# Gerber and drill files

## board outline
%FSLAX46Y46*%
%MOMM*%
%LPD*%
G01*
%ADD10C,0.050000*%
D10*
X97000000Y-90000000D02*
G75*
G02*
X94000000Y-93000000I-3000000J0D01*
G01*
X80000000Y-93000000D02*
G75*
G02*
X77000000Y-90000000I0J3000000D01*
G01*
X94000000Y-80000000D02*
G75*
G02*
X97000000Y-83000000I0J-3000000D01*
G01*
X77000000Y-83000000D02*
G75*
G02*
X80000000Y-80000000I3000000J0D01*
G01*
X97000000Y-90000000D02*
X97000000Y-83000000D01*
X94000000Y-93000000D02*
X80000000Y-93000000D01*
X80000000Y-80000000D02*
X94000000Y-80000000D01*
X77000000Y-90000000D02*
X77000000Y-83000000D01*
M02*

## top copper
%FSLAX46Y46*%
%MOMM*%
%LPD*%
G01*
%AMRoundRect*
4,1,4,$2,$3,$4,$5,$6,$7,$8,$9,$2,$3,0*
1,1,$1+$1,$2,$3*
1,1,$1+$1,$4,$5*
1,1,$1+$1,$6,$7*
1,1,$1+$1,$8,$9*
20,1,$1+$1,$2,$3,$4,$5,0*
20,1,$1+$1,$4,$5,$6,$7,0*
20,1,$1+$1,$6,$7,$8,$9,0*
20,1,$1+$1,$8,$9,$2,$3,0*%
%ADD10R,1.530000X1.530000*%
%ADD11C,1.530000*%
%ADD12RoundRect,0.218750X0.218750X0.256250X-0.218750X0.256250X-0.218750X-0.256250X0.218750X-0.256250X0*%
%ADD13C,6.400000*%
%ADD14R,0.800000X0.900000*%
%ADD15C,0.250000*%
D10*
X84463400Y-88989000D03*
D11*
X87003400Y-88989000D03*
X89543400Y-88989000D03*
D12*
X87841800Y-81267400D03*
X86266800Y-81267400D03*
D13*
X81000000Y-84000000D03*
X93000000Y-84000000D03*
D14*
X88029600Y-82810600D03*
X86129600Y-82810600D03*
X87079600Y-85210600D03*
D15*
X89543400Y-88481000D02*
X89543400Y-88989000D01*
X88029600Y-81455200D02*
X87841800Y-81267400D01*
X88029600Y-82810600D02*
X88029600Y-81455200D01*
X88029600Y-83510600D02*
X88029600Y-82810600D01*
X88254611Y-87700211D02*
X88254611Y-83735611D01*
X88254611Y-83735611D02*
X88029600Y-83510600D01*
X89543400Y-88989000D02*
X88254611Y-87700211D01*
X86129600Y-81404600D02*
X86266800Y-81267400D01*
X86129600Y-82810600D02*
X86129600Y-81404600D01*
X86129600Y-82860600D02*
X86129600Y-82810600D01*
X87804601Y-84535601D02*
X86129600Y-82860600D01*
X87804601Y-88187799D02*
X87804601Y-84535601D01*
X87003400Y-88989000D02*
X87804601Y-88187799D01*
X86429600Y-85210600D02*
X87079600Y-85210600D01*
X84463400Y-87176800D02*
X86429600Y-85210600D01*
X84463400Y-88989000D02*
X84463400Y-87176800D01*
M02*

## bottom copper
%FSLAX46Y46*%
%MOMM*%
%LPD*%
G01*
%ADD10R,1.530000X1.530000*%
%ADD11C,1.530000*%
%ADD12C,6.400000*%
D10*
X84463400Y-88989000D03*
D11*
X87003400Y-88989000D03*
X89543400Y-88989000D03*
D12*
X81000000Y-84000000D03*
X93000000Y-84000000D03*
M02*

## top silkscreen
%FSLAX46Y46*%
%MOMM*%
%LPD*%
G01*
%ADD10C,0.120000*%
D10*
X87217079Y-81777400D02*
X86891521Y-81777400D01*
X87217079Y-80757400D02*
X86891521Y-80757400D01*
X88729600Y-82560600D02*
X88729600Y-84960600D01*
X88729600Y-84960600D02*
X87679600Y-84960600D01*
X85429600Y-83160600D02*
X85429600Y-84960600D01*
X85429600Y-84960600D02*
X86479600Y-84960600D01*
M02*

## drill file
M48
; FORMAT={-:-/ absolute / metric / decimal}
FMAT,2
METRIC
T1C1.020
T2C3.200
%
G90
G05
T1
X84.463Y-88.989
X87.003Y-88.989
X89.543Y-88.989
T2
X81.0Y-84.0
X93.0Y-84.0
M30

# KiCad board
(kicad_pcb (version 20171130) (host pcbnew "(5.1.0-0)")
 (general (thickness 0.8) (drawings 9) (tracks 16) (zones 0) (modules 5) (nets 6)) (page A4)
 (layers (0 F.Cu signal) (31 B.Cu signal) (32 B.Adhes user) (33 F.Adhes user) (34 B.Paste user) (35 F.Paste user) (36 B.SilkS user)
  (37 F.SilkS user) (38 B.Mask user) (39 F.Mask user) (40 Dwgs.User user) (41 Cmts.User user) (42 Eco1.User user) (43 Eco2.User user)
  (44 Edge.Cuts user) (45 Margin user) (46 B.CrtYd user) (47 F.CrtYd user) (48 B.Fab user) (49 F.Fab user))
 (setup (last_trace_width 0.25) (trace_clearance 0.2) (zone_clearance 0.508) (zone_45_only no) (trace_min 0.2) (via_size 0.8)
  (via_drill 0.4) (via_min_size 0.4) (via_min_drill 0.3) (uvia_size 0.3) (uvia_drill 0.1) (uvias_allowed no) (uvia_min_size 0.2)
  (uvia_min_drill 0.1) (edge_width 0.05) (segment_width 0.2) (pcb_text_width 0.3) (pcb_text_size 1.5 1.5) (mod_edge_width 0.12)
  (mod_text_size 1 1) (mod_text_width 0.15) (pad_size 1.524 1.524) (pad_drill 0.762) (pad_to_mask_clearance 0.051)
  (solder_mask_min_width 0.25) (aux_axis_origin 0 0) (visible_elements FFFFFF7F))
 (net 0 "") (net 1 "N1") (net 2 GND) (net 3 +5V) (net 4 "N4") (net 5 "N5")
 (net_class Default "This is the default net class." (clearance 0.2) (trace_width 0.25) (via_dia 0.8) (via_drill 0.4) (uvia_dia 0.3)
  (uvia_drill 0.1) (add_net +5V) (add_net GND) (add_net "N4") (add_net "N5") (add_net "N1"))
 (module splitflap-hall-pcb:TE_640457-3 (layer B.Cu) (at 84.4634 88.989 180)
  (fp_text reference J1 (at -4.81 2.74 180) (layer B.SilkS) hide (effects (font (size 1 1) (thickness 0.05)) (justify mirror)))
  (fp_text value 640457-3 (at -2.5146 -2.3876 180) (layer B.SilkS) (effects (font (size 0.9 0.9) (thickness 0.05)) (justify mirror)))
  (pad 1 thru_hole rect (at 0 0 180) (size 1.53 1.53) (drill 1.02) (layers *.Cu *.Mask) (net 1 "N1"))
  (pad 2 thru_hole circle (at -2.54 0 180) (size 1.53 1.53) (drill 1.02) (layers *.Cu *.Mask) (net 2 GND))
  (pad 3 thru_hole circle (at -5.08 0 180) (size 1.53 1.53) (drill 1.02) (layers *.Cu *.Mask) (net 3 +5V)))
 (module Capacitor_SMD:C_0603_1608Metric (layer F.Cu) (at 87.0543 81.2674 180)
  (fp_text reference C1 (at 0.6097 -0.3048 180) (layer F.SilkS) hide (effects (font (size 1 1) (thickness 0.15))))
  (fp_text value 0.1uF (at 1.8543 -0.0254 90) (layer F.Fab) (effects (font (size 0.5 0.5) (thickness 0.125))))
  (fp_line (start -0.162779 -0.51) (end 0.162779 -0.51) (layer F.SilkS) (width 0.12))
  (fp_line (start -0.162779 0.51) (end 0.162779 0.51) (layer F.SilkS) (width 0.12))
  (pad 1 smd roundrect (at -0.7875 0 180) (size 0.875 0.95) (layers F.Cu F.Paste F.Mask) (roundrect_rratio 0.25) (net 3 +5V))
  (pad 2 smd roundrect (at 0.7875 0 180) (size 0.875 0.95) (layers F.Cu F.Paste F.Mask) (roundrect_rratio 0.25) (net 2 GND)))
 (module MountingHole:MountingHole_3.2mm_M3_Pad (layer F.Cu) (at 81 84 90)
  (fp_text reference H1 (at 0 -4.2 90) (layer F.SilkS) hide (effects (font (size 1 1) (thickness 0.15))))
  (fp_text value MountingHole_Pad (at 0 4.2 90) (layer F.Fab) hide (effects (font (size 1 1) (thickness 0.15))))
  (pad 1 thru_hole circle (at 0 0 90) (size 6.4 6.4) (drill 3.2) (layers *.Cu *.Mask) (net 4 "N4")))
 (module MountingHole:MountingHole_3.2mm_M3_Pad (layer F.Cu) (at 93 84 90)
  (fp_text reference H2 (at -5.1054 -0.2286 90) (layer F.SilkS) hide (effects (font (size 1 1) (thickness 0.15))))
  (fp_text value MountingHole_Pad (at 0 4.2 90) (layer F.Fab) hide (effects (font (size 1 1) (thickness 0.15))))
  (pad 1 thru_hole circle (at 0 0 90) (size 6.4 6.4) (drill 3.2) (layers *.Cu *.Mask) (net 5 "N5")))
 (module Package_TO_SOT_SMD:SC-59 (layer F.Cu) (at 87.0796 84.0106 270)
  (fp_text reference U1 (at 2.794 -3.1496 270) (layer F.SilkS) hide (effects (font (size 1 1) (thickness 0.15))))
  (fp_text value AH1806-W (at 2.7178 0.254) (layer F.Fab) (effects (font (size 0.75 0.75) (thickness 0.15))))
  (fp_line (start -1.45 -1.65) (end 0.95 -1.65) (layer F.SilkS) (width 0.12))
  (fp_line (start 0.95 -1.65) (end 0.95 -0.6) (layer F.SilkS) (width 0.12))
  (fp_line (start -0.85 1.65) (end 0.95 1.65) (layer F.SilkS) (width 0.12))
  (fp_line (start 0.95 1.65) (end 0.95 0.6) (layer F.SilkS) (width 0.12))
  (pad 1 smd rect (at -1.2 -0.95 270) (size 0.9 0.8) (layers F.Cu F.Paste F.Mask) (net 3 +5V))
  (pad 2 smd rect (at -1.2 0.95 270) (size 0.9 0.8) (layers F.Cu F.Paste F.Mask) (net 2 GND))
  (pad 3 smd rect (at 1.2 0 270) (size 0.9 0.8) (layers F.Cu F.Paste F.Mask) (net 1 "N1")))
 (gr_arc (start 94 90) (end 97 90) (angle 90) (layer Edge.Cuts) (width 0.05))
 (gr_arc (start 80 90) (end 80 93) (angle 90) (layer Edge.Cuts) (width 0.05))
 (gr_arc (start 94 83) (end 94 80) (angle 90) (layer Edge.Cuts) (width 0.05))
 (gr_arc (start 80 83) (end 77 83) (angle 90) (layer Edge.Cuts) (width 0.05))
 (gr_line (start 97 90) (end 97 83) (layer Edge.Cuts) (width 0.05))
 (gr_line (start 94 93) (end 80 93) (layer Edge.Cuts) (width 0.05))
 (gr_line (start 80 80) (end 94 80) (layer Edge.Cuts) (width 0.05))
 (gr_line (start 77 90) (end 77 83) (layer Edge.Cuts) (width 0.05))
 (segment (start 89.5434 88.481) (end 89.5434 88.989) (width 0.25) (layer F.Cu) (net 3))
 (segment (start 88.0296 81.4552) (end 87.8418 81.2674) (width 0.25) (layer F.Cu) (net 3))
 (segment (start 88.0296 82.8106) (end 88.0296 81.4552) (width 0.25) (layer F.Cu) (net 3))
 (segment (start 88.0296 83.5106) (end 88.0296 82.8106) (width 0.25) (layer F.Cu) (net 3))
 (segment (start 88.254611 87.700211) (end 88.254611 83.735611) (width 0.25) (layer F.Cu) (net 3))
 (segment (start 88.254611 83.735611) (end 88.0296 83.5106) (width 0.25) (layer F.Cu) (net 3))
 (segment (start 89.5434 88.989) (end 88.254611 87.700211) (width 0.25) (layer F.Cu) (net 3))
 (segment (start 86.1296 81.4046) (end 86.2668 81.2674) (width 0.25) (layer F.Cu) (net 2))
 (segment (start 86.1296 82.8106) (end 86.1296 81.4046) (width 0.25) (layer F.Cu) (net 2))
 (segment (start 86.1296 82.8606) (end 86.1296 82.8106) (width 0.25) (layer F.Cu) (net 2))
 (segment (start 87.804601 84.535601) (end 86.1296 82.8606) (width 0.25) (layer F.Cu) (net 2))
 (segment (start 87.804601 88.187799) (end 87.804601 84.535601) (width 0.25) (layer F.Cu) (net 2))
 (segment (start 87.0034 88.989) (end 87.804601 88.187799) (width 0.25) (layer F.Cu) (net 2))
 (segment (start 86.4296 85.2106) (end 87.0796 85.2106) (width 0.25) (layer F.Cu) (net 1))
 (segment (start 84.4634 87.1768) (end 86.4296 85.2106) (width 0.25) (layer F.Cu) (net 1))
 (segment (start 84.4634 88.989) (end 84.4634 87.1768) (width 0.25) (layer F.Cu) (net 1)))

